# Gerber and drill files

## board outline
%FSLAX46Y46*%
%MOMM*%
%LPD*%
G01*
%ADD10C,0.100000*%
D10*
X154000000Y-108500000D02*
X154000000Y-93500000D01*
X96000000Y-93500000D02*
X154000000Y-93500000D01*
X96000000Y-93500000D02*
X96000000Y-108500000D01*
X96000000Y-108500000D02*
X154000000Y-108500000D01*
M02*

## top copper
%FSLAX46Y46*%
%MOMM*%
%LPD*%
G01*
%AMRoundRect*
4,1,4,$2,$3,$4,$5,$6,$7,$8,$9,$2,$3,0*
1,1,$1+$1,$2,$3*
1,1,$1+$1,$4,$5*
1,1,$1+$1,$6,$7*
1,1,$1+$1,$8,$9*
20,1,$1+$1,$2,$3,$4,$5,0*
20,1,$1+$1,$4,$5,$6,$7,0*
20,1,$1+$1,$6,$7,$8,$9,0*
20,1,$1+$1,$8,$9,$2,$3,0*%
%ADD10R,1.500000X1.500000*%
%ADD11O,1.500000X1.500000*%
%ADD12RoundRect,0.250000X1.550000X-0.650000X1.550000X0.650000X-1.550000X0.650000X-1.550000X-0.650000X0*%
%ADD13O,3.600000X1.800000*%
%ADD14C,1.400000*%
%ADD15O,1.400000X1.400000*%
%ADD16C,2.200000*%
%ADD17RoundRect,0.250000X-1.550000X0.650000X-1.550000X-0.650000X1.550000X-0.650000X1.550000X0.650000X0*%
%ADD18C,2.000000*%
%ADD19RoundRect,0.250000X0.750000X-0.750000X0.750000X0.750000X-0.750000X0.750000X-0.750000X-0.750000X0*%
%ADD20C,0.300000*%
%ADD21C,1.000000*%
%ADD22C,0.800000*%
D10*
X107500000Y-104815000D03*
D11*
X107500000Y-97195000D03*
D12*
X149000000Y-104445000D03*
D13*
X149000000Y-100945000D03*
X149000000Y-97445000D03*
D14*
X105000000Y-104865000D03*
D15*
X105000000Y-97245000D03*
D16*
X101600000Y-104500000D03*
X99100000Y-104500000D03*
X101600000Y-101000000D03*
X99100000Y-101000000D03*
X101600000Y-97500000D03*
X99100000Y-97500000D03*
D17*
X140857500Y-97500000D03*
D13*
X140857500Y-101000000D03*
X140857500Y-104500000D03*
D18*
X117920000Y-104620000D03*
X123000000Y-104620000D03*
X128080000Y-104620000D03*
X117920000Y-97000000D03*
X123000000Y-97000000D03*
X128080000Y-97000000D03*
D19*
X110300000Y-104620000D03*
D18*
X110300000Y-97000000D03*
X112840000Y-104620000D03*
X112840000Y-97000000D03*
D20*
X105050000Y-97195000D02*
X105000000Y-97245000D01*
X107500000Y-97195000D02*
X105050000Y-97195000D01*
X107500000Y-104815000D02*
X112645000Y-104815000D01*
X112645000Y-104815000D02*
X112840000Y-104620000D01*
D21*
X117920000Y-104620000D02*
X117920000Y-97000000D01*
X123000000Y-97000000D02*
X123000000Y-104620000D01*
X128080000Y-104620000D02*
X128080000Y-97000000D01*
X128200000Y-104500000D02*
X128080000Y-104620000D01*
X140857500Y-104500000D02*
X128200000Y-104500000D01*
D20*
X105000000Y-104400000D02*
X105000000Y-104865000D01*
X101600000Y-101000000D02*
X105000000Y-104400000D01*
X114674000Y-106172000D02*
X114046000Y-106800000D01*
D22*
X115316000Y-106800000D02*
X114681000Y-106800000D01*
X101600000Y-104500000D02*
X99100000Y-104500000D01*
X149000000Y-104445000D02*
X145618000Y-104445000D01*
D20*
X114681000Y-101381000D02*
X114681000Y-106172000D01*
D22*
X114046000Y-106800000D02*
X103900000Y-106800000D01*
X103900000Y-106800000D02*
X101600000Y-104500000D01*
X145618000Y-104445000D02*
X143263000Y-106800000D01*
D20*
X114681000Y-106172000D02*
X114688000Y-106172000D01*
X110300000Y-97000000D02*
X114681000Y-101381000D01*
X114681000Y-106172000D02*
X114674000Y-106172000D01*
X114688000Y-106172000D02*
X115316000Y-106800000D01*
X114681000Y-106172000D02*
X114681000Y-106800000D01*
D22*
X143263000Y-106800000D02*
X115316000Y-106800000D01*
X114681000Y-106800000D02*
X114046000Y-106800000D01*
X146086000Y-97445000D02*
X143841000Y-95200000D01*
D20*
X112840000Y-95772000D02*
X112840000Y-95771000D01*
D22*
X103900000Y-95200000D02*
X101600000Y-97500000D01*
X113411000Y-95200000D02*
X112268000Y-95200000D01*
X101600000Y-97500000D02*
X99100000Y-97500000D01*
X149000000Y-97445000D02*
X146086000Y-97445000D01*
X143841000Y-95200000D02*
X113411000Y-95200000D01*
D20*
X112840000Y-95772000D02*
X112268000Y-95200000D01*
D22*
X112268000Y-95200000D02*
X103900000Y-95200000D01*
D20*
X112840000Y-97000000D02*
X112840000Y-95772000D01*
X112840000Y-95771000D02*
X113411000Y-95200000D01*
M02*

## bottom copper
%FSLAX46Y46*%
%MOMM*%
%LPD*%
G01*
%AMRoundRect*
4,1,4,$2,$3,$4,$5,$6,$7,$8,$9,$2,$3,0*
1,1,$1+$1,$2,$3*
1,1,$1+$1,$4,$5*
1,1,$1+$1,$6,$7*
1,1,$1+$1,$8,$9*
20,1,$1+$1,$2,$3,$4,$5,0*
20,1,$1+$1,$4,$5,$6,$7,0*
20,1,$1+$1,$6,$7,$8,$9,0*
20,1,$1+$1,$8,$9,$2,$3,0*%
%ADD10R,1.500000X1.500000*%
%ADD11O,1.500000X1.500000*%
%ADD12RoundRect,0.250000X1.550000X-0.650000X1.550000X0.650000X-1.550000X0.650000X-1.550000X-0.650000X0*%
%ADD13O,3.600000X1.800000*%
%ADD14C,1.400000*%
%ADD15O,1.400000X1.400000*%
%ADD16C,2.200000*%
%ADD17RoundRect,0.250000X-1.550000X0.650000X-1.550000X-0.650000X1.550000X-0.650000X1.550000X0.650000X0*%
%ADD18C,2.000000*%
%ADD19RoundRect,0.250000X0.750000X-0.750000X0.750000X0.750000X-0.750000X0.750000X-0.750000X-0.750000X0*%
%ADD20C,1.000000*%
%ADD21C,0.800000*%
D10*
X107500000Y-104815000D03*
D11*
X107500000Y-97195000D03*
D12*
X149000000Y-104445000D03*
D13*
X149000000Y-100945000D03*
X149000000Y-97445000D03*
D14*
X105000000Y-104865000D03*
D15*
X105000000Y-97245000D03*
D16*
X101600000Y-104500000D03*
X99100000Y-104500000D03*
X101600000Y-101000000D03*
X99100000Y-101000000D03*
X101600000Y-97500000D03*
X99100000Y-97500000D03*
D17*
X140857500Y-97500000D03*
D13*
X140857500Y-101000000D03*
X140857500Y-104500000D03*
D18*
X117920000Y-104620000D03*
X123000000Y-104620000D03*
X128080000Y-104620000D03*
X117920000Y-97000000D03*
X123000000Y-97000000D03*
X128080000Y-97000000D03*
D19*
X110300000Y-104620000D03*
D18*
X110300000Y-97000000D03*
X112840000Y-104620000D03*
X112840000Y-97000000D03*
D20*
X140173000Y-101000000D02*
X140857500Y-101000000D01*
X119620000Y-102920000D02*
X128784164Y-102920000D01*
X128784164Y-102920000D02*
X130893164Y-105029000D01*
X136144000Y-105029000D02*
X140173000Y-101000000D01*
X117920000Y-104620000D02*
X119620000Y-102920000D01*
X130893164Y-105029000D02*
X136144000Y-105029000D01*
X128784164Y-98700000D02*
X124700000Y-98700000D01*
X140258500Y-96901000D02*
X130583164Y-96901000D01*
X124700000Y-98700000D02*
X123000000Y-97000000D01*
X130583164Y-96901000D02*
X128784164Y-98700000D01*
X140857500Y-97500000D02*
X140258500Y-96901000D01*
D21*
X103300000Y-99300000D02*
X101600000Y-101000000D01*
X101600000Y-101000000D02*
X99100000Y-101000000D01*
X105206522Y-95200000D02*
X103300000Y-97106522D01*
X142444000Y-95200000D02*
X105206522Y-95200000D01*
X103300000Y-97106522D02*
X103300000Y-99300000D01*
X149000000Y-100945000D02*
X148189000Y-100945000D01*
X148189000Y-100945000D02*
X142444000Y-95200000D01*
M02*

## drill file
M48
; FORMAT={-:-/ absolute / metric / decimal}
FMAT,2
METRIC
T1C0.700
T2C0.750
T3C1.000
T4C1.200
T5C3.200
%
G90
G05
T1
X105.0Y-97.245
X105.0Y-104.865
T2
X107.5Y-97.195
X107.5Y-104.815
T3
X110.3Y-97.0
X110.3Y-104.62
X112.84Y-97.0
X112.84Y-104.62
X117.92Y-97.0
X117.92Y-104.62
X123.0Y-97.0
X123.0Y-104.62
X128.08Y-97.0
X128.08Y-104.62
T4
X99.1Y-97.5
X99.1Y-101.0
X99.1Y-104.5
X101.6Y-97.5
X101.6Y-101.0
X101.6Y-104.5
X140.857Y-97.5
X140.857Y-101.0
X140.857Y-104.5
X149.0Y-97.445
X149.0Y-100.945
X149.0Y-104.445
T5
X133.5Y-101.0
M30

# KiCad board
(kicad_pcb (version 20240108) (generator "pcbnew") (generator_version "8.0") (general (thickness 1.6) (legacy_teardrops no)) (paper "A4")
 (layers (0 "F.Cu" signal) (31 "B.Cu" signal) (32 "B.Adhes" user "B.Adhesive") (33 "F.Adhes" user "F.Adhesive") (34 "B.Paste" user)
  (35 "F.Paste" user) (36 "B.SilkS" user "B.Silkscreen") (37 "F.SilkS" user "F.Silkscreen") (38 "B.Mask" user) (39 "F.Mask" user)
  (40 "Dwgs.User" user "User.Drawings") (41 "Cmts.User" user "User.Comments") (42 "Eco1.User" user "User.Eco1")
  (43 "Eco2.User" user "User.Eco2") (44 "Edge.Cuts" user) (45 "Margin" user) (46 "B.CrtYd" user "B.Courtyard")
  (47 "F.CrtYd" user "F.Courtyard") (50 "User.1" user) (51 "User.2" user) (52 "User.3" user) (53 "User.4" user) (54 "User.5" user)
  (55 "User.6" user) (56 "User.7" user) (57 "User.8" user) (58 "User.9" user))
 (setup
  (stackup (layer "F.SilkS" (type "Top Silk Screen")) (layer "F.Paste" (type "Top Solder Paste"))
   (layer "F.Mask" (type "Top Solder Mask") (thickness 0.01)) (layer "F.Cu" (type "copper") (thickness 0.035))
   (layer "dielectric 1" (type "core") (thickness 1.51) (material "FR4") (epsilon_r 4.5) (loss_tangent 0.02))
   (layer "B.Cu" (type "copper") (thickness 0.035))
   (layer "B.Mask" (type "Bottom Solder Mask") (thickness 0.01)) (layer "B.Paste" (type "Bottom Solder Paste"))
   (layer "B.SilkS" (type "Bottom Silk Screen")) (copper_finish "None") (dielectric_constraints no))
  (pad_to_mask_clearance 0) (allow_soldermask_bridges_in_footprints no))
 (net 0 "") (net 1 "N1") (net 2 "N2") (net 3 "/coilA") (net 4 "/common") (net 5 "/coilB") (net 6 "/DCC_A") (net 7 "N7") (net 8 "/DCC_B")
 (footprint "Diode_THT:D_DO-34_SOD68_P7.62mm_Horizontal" (layer "F.Cu") (at 107.5 104.815 90)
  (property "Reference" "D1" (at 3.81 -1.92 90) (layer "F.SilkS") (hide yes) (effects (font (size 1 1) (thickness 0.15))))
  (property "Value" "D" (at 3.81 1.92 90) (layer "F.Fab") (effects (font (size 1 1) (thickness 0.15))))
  (pad "1" thru_hole rect (at 0 0 90) (size 1.5 1.5) (drill 0.75) (layers "*.Cu" "*.Mask") (remove_unused_layers no) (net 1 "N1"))
  (pad "2" thru_hole oval (at 7.62 0 90) (size 1.5 1.5) (drill 0.75) (layers "*.Cu" "*.Mask") (remove_unused_layers no) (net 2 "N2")))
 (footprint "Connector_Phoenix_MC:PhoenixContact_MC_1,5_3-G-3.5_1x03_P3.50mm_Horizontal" (layer "F.Cu") (at 149 104.445 90)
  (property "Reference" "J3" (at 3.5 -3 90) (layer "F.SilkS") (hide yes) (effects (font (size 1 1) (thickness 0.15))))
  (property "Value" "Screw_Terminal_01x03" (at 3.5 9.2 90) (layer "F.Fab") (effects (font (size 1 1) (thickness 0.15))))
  (pad "1" thru_hole roundrect (at 0 0 90) (size 1.8 3.6) (drill 1.2) (layers "*.Cu" "*.Mask") (remove_unused_layers no)
   (roundrect_rratio 0.138889) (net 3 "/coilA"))
  (pad "2" thru_hole oval (at 3.5 0 90) (size 1.8 3.6) (drill 1.2) (layers "*.Cu" "*.Mask") (remove_unused_layers no) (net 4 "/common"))
  (pad "3" thru_hole oval (at 7 0 90) (size 1.8 3.6) (drill 1.2) (layers "*.Cu" "*.Mask") (remove_unused_layers no) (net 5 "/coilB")))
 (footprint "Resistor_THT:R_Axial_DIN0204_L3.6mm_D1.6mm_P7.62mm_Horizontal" (layer "F.Cu") (at 105 104.865 90)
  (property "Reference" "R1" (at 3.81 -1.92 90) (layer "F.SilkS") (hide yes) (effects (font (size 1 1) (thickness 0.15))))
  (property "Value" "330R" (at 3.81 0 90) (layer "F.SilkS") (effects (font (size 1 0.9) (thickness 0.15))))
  (pad "1" thru_hole circle (at 0 0 90) (size 1.4 1.4) (drill 0.7) (layers "*.Cu" "*.Mask") (remove_unused_layers no) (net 4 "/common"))
  (pad "2" thru_hole oval (at 7.62 0 90) (size 1.4 1.4) (drill 0.7) (layers "*.Cu" "*.Mask") (remove_unused_layers no) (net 2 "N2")))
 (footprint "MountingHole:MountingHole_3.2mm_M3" (layer "F.Cu") (at 133.5 101)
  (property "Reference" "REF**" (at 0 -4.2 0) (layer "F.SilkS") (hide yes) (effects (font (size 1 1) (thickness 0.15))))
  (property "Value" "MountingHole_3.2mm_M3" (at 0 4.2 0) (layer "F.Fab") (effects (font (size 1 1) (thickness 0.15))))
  (pad "" np_thru_hole circle (at 0 0) (size 3.2 3.2) (drill 3.2) (layers "*.Cu" "*.Mask")))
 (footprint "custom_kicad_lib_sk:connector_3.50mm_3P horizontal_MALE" (layer "F.Cu") (at 101.6 101 -90)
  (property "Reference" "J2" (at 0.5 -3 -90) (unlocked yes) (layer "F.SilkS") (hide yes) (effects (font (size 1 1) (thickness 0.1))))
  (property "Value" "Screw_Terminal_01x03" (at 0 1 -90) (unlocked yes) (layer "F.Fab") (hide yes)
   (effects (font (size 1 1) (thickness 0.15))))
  (pad "1" thru_hole circle (at 3.5 0 270) (size 2.2 2.2) (drill 1.2) (layers "*.Cu" "*.Mask") (remove_unused_layers no) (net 3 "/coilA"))
  (pad "1" thru_hole circle (at 3.5 2.5 270) (size 2.2 2.2) (drill 1.2) (layers "*.Cu" "*.Mask") (remove_unused_layers no) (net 3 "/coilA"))
  (pad "2" thru_hole circle (at 0 0 270) (size 2.2 2.2) (drill 1.2) (layers "*.Cu" "*.Mask") (remove_unused_layers no) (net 4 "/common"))
  (pad "2" thru_hole circle (at 0 2.5 270) (size 2.2 2.2) (drill 1.2) (layers "*.Cu" "*.Mask") (remove_unused_layers no) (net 4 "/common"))
  (pad "3" thru_hole circle (at -3.5 0 270) (size 2.2 2.2) (drill 1.2) (layers "*.Cu" "*.Mask") (remove_unused_layers no) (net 5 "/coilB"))
  (pad "3" thru_hole circle (at -3.5 2.5 270) (size 2.2 2.2) (drill 1.2) (layers "*.Cu" "*.Mask") (remove_unused_layers no) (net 5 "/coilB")))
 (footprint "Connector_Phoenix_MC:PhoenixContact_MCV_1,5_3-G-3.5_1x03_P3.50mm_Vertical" (layer "F.Cu") (at 140.8575 97.5 -90)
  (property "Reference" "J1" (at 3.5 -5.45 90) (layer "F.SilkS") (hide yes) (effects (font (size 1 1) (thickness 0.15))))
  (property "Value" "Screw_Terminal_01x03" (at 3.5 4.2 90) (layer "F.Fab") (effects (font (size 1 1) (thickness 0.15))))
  (pad "1" thru_hole roundrect (at 0 0 270) (size 1.8 3.6) (drill 1.2) (layers "*.Cu" "*.Mask") (remove_unused_layers no)
   (roundrect_rratio 0.138889) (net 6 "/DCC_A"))
  (pad "2" thru_hole oval (at 3.5 0 270) (size 1.8 3.6) (drill 1.2) (layers "*.Cu" "*.Mask") (remove_unused_layers no) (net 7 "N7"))
  (pad "3" thru_hole oval (at 7 0 270) (size 1.8 3.6) (drill 1.2) (layers "*.Cu" "*.Mask") (remove_unused_layers no) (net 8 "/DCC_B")))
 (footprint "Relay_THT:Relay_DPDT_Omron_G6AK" (layer "F.Cu") (at 110.3 104.62 90)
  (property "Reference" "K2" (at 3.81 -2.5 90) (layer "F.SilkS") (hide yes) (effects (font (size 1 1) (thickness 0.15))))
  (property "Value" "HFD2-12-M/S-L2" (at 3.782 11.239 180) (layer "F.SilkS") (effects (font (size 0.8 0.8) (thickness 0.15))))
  (pad "11" thru_hole circle (at 0 7.62 90) (size 2 2) (drill 1) (layers "*.Cu" "*.Mask") (remove_unused_layers no) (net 7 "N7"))
  (pad "12" thru_hole circle (at 0 12.7 90) (size 2 2) (drill 1) (layers "*.Cu" "*.Mask") (remove_unused_layers no) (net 6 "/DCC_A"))
  (pad "14" thru_hole circle (at 0 17.78 90) (size 2 2) (drill 1) (layers "*.Cu" "*.Mask") (remove_unused_layers no) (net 8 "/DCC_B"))
  (pad "21" thru_hole circle (at 7.62 7.62 90) (size 2 2) (drill 1) (layers "*.Cu" "*.Mask") (remove_unused_layers no) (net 7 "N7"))
  (pad "22" thru_hole circle (at 7.62 12.7 90) (size 2 2) (drill 1) (layers "*.Cu" "*.Mask") (remove_unused_layers no) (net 6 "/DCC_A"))
  (pad "24" thru_hole circle (at 7.62 17.78 90) (size 2 2) (drill 1) (layers "*.Cu" "*.Mask") (remove_unused_layers no) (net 8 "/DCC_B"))
  (pad "A1" thru_hole roundrect (at 0 0 90) (size 2 2) (drill 1) (layers "*.Cu" "*.Mask") (remove_unused_layers no) (roundrect_rratio 0.125)
   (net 1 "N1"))
  (pad "A2" thru_hole circle (at 7.62 0 90) (size 2 2) (drill 1) (layers "*.Cu" "*.Mask") (remove_unused_layers no) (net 3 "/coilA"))
  (pad "B1" thru_hole circle (at 0 2.54 90) (size 2 2) (drill 1) (layers "*.Cu" "*.Mask") (remove_unused_layers no) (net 1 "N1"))
  (pad "B2" thru_hole circle (at 7.62 2.54 90) (size 2 2) (drill 1) (layers "*.Cu" "*.Mask") (remove_unused_layers no) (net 5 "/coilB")))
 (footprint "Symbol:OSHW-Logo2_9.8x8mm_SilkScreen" (layer "B.Cu") (at 116.5 100.838 -90)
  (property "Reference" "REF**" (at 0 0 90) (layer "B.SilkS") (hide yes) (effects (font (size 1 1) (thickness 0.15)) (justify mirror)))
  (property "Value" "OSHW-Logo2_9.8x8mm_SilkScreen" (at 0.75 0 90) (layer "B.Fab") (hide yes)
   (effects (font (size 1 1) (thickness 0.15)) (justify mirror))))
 (gr_line (start 154 108.5) (end 154 93.5) (stroke (width 0.1) (type default)) (layer "Edge.Cuts"))
 (gr_line (start 96 93.5) (end 154 93.5) (stroke (width 0.1) (type default)) (layer "Edge.Cuts"))
 (gr_line (start 96 93.5) (end 96 108.5) (stroke (width 0.1) (type default)) (layer "Edge.Cuts"))
 (gr_line (start 96 108.5) (end 154 108.5) (stroke (width 0.1) (type default)) (layer "Edge.Cuts"))
 (segment (start 105.05 97.195) (end 105 97.245) (width 0.3) (layer "F.Cu") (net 2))
 (segment (start 107.5 97.195) (end 105.05 97.195) (width 0.3) (layer "F.Cu") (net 2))
 (segment (start 107.5 104.815) (end 112.645 104.815) (width 0.3) (layer "F.Cu") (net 1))
 (segment (start 112.645 104.815) (end 112.84 104.62) (width 0.3) (layer "F.Cu") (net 1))
 (segment (start 117.92 104.62) (end 117.92 97) (width 1) (layer "F.Cu") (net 7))
 (segment (start 140.173 101) (end 140.8575 101) (width 1) (layer "B.Cu") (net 7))
 (segment (start 119.62 102.92) (end 128.784164 102.92) (width 1) (layer "B.Cu") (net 7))
 (segment (start 128.784164 102.92) (end 130.893164 105.029) (width 1) (layer "B.Cu") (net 7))
 (segment (start 136.144 105.029) (end 140.173 101) (width 1) (layer "B.Cu") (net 7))
 (segment (start 117.92 104.62) (end 119.62 102.92) (width 1) (layer "B.Cu") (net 7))
 (segment (start 130.893164 105.029) (end 136.144 105.029) (width 1) (layer "B.Cu") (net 7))
 (segment (start 123 97) (end 123 104.62) (width 1) (layer "F.Cu") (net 6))
 (segment (start 128.784164 98.7) (end 124.7 98.7) (width 1) (layer "B.Cu") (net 6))
 (segment (start 140.2585 96.901) (end 130.583164 96.901) (width 1) (layer "B.Cu") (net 6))
 (segment (start 124.7 98.7) (end 123 97) (width 1) (layer "B.Cu") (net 6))
 (segment (start 130.583164 96.901) (end 128.784164 98.7) (width 1) (layer "B.Cu") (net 6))
 (segment (start 140.8575 97.5) (end 140.2585 96.901) (width 1) (layer "B.Cu") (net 6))
 (segment (start 128.08 104.62) (end 128.08 97) (width 1) (layer "F.Cu") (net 8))
 (segment (start 128.2 104.5) (end 128.08 104.62) (width 1) (layer "F.Cu") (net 8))
 (segment (start 140.8575 104.5) (end 128.2 104.5) (width 1) (layer "F.Cu") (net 8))
 (segment (start 105 104.4) (end 105 104.865) (width 0.3) (layer "F.Cu") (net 4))
 (segment (start 101.6 101) (end 105 104.4) (width 0.3) (layer "F.Cu") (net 4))
 (segment (start 103.3 99.3) (end 101.6 101) (width 0.8) (layer "B.Cu") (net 4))
 (segment (start 101.6 101) (end 99.1 101) (width 0.8) (layer "B.Cu") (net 4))
 (segment (start 105.206522 95.2) (end 103.3 97.106522) (width 0.8) (layer "B.Cu") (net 4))
 (segment (start 142.444 95.2) (end 105.206522 95.2) (width 0.8) (layer "B.Cu") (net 4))
 (segment (start 103.3 97.106522) (end 103.3 99.3) (width 0.8) (layer "B.Cu") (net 4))
 (segment (start 149 100.945) (end 148.189 100.945) (width 0.8) (layer "B.Cu") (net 4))
 (segment (start 148.189 100.945) (end 142.444 95.2) (width 0.8) (layer "B.Cu") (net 4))
 (segment (start 114.674 106.172) (end 114.046 106.8) (width 0.3) (layer "F.Cu") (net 3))
 (segment (start 115.316 106.8) (end 114.681 106.8) (width 0.8) (layer "F.Cu") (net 3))
 (segment (start 101.6 104.5) (end 99.1 104.5) (width 0.8) (layer "F.Cu") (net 3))
 (segment (start 149 104.445) (end 145.618 104.445) (width 0.8) (layer "F.Cu") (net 3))
 (segment (start 114.681 101.381) (end 114.681 106.172) (width 0.3) (layer "F.Cu") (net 3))
 (segment (start 114.046 106.8) (end 103.9 106.8) (width 0.8) (layer "F.Cu") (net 3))
 (segment (start 103.9 106.8) (end 101.6 104.5) (width 0.8) (layer "F.Cu") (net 3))
 (segment (start 145.618 104.445) (end 143.263 106.8) (width 0.8) (layer "F.Cu") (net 3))
 (segment (start 114.681 106.172) (end 114.688 106.172) (width 0.3) (layer "F.Cu") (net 3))
 (segment (start 110.3 97) (end 114.681 101.381) (width 0.3) (layer "F.Cu") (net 3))
 (segment (start 114.681 106.172) (end 114.674 106.172) (width 0.3) (layer "F.Cu") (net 3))
 (segment (start 114.688 106.172) (end 115.316 106.8) (width 0.3) (layer "F.Cu") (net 3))
 (segment (start 114.681 106.172) (end 114.681 106.8) (width 0.3) (layer "F.Cu") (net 3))
 (segment (start 143.263 106.8) (end 115.316 106.8) (width 0.8) (layer "F.Cu") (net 3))
 (segment (start 114.681 106.8) (end 114.046 106.8) (width 0.8) (layer "F.Cu") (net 3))
 (segment (start 146.086 97.445) (end 143.841 95.2) (width 0.8) (layer "F.Cu") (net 5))
 (segment (start 112.84 95.772) (end 112.84 95.771) (width 0.3) (layer "F.Cu") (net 5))
 (segment (start 103.9 95.2) (end 101.6 97.5) (width 0.8) (layer "F.Cu") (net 5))
 (segment (start 113.411 95.2) (end 112.268 95.2) (width 0.8) (layer "F.Cu") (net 5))
 (segment (start 101.6 97.5) (end 99.1 97.5) (width 0.8) (layer "F.Cu") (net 5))
 (segment (start 149 97.445) (end 146.086 97.445) (width 0.8) (layer "F.Cu") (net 5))
 (segment (start 143.841 95.2) (end 113.411 95.2) (width 0.8) (layer "F.Cu") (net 5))
 (segment (start 112.84 95.772) (end 112.268 95.2) (width 0.3) (layer "F.Cu") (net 5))
 (segment (start 112.268 95.2) (end 103.9 95.2) (width 0.8) (layer "F.Cu") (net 5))
 (segment (start 112.84 97) (end 112.84 95.772) (width 0.3) (layer "F.Cu") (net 5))
 (segment (start 112.84 95.771) (end 113.411 95.2) (width 0.3) (layer "F.Cu") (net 5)))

